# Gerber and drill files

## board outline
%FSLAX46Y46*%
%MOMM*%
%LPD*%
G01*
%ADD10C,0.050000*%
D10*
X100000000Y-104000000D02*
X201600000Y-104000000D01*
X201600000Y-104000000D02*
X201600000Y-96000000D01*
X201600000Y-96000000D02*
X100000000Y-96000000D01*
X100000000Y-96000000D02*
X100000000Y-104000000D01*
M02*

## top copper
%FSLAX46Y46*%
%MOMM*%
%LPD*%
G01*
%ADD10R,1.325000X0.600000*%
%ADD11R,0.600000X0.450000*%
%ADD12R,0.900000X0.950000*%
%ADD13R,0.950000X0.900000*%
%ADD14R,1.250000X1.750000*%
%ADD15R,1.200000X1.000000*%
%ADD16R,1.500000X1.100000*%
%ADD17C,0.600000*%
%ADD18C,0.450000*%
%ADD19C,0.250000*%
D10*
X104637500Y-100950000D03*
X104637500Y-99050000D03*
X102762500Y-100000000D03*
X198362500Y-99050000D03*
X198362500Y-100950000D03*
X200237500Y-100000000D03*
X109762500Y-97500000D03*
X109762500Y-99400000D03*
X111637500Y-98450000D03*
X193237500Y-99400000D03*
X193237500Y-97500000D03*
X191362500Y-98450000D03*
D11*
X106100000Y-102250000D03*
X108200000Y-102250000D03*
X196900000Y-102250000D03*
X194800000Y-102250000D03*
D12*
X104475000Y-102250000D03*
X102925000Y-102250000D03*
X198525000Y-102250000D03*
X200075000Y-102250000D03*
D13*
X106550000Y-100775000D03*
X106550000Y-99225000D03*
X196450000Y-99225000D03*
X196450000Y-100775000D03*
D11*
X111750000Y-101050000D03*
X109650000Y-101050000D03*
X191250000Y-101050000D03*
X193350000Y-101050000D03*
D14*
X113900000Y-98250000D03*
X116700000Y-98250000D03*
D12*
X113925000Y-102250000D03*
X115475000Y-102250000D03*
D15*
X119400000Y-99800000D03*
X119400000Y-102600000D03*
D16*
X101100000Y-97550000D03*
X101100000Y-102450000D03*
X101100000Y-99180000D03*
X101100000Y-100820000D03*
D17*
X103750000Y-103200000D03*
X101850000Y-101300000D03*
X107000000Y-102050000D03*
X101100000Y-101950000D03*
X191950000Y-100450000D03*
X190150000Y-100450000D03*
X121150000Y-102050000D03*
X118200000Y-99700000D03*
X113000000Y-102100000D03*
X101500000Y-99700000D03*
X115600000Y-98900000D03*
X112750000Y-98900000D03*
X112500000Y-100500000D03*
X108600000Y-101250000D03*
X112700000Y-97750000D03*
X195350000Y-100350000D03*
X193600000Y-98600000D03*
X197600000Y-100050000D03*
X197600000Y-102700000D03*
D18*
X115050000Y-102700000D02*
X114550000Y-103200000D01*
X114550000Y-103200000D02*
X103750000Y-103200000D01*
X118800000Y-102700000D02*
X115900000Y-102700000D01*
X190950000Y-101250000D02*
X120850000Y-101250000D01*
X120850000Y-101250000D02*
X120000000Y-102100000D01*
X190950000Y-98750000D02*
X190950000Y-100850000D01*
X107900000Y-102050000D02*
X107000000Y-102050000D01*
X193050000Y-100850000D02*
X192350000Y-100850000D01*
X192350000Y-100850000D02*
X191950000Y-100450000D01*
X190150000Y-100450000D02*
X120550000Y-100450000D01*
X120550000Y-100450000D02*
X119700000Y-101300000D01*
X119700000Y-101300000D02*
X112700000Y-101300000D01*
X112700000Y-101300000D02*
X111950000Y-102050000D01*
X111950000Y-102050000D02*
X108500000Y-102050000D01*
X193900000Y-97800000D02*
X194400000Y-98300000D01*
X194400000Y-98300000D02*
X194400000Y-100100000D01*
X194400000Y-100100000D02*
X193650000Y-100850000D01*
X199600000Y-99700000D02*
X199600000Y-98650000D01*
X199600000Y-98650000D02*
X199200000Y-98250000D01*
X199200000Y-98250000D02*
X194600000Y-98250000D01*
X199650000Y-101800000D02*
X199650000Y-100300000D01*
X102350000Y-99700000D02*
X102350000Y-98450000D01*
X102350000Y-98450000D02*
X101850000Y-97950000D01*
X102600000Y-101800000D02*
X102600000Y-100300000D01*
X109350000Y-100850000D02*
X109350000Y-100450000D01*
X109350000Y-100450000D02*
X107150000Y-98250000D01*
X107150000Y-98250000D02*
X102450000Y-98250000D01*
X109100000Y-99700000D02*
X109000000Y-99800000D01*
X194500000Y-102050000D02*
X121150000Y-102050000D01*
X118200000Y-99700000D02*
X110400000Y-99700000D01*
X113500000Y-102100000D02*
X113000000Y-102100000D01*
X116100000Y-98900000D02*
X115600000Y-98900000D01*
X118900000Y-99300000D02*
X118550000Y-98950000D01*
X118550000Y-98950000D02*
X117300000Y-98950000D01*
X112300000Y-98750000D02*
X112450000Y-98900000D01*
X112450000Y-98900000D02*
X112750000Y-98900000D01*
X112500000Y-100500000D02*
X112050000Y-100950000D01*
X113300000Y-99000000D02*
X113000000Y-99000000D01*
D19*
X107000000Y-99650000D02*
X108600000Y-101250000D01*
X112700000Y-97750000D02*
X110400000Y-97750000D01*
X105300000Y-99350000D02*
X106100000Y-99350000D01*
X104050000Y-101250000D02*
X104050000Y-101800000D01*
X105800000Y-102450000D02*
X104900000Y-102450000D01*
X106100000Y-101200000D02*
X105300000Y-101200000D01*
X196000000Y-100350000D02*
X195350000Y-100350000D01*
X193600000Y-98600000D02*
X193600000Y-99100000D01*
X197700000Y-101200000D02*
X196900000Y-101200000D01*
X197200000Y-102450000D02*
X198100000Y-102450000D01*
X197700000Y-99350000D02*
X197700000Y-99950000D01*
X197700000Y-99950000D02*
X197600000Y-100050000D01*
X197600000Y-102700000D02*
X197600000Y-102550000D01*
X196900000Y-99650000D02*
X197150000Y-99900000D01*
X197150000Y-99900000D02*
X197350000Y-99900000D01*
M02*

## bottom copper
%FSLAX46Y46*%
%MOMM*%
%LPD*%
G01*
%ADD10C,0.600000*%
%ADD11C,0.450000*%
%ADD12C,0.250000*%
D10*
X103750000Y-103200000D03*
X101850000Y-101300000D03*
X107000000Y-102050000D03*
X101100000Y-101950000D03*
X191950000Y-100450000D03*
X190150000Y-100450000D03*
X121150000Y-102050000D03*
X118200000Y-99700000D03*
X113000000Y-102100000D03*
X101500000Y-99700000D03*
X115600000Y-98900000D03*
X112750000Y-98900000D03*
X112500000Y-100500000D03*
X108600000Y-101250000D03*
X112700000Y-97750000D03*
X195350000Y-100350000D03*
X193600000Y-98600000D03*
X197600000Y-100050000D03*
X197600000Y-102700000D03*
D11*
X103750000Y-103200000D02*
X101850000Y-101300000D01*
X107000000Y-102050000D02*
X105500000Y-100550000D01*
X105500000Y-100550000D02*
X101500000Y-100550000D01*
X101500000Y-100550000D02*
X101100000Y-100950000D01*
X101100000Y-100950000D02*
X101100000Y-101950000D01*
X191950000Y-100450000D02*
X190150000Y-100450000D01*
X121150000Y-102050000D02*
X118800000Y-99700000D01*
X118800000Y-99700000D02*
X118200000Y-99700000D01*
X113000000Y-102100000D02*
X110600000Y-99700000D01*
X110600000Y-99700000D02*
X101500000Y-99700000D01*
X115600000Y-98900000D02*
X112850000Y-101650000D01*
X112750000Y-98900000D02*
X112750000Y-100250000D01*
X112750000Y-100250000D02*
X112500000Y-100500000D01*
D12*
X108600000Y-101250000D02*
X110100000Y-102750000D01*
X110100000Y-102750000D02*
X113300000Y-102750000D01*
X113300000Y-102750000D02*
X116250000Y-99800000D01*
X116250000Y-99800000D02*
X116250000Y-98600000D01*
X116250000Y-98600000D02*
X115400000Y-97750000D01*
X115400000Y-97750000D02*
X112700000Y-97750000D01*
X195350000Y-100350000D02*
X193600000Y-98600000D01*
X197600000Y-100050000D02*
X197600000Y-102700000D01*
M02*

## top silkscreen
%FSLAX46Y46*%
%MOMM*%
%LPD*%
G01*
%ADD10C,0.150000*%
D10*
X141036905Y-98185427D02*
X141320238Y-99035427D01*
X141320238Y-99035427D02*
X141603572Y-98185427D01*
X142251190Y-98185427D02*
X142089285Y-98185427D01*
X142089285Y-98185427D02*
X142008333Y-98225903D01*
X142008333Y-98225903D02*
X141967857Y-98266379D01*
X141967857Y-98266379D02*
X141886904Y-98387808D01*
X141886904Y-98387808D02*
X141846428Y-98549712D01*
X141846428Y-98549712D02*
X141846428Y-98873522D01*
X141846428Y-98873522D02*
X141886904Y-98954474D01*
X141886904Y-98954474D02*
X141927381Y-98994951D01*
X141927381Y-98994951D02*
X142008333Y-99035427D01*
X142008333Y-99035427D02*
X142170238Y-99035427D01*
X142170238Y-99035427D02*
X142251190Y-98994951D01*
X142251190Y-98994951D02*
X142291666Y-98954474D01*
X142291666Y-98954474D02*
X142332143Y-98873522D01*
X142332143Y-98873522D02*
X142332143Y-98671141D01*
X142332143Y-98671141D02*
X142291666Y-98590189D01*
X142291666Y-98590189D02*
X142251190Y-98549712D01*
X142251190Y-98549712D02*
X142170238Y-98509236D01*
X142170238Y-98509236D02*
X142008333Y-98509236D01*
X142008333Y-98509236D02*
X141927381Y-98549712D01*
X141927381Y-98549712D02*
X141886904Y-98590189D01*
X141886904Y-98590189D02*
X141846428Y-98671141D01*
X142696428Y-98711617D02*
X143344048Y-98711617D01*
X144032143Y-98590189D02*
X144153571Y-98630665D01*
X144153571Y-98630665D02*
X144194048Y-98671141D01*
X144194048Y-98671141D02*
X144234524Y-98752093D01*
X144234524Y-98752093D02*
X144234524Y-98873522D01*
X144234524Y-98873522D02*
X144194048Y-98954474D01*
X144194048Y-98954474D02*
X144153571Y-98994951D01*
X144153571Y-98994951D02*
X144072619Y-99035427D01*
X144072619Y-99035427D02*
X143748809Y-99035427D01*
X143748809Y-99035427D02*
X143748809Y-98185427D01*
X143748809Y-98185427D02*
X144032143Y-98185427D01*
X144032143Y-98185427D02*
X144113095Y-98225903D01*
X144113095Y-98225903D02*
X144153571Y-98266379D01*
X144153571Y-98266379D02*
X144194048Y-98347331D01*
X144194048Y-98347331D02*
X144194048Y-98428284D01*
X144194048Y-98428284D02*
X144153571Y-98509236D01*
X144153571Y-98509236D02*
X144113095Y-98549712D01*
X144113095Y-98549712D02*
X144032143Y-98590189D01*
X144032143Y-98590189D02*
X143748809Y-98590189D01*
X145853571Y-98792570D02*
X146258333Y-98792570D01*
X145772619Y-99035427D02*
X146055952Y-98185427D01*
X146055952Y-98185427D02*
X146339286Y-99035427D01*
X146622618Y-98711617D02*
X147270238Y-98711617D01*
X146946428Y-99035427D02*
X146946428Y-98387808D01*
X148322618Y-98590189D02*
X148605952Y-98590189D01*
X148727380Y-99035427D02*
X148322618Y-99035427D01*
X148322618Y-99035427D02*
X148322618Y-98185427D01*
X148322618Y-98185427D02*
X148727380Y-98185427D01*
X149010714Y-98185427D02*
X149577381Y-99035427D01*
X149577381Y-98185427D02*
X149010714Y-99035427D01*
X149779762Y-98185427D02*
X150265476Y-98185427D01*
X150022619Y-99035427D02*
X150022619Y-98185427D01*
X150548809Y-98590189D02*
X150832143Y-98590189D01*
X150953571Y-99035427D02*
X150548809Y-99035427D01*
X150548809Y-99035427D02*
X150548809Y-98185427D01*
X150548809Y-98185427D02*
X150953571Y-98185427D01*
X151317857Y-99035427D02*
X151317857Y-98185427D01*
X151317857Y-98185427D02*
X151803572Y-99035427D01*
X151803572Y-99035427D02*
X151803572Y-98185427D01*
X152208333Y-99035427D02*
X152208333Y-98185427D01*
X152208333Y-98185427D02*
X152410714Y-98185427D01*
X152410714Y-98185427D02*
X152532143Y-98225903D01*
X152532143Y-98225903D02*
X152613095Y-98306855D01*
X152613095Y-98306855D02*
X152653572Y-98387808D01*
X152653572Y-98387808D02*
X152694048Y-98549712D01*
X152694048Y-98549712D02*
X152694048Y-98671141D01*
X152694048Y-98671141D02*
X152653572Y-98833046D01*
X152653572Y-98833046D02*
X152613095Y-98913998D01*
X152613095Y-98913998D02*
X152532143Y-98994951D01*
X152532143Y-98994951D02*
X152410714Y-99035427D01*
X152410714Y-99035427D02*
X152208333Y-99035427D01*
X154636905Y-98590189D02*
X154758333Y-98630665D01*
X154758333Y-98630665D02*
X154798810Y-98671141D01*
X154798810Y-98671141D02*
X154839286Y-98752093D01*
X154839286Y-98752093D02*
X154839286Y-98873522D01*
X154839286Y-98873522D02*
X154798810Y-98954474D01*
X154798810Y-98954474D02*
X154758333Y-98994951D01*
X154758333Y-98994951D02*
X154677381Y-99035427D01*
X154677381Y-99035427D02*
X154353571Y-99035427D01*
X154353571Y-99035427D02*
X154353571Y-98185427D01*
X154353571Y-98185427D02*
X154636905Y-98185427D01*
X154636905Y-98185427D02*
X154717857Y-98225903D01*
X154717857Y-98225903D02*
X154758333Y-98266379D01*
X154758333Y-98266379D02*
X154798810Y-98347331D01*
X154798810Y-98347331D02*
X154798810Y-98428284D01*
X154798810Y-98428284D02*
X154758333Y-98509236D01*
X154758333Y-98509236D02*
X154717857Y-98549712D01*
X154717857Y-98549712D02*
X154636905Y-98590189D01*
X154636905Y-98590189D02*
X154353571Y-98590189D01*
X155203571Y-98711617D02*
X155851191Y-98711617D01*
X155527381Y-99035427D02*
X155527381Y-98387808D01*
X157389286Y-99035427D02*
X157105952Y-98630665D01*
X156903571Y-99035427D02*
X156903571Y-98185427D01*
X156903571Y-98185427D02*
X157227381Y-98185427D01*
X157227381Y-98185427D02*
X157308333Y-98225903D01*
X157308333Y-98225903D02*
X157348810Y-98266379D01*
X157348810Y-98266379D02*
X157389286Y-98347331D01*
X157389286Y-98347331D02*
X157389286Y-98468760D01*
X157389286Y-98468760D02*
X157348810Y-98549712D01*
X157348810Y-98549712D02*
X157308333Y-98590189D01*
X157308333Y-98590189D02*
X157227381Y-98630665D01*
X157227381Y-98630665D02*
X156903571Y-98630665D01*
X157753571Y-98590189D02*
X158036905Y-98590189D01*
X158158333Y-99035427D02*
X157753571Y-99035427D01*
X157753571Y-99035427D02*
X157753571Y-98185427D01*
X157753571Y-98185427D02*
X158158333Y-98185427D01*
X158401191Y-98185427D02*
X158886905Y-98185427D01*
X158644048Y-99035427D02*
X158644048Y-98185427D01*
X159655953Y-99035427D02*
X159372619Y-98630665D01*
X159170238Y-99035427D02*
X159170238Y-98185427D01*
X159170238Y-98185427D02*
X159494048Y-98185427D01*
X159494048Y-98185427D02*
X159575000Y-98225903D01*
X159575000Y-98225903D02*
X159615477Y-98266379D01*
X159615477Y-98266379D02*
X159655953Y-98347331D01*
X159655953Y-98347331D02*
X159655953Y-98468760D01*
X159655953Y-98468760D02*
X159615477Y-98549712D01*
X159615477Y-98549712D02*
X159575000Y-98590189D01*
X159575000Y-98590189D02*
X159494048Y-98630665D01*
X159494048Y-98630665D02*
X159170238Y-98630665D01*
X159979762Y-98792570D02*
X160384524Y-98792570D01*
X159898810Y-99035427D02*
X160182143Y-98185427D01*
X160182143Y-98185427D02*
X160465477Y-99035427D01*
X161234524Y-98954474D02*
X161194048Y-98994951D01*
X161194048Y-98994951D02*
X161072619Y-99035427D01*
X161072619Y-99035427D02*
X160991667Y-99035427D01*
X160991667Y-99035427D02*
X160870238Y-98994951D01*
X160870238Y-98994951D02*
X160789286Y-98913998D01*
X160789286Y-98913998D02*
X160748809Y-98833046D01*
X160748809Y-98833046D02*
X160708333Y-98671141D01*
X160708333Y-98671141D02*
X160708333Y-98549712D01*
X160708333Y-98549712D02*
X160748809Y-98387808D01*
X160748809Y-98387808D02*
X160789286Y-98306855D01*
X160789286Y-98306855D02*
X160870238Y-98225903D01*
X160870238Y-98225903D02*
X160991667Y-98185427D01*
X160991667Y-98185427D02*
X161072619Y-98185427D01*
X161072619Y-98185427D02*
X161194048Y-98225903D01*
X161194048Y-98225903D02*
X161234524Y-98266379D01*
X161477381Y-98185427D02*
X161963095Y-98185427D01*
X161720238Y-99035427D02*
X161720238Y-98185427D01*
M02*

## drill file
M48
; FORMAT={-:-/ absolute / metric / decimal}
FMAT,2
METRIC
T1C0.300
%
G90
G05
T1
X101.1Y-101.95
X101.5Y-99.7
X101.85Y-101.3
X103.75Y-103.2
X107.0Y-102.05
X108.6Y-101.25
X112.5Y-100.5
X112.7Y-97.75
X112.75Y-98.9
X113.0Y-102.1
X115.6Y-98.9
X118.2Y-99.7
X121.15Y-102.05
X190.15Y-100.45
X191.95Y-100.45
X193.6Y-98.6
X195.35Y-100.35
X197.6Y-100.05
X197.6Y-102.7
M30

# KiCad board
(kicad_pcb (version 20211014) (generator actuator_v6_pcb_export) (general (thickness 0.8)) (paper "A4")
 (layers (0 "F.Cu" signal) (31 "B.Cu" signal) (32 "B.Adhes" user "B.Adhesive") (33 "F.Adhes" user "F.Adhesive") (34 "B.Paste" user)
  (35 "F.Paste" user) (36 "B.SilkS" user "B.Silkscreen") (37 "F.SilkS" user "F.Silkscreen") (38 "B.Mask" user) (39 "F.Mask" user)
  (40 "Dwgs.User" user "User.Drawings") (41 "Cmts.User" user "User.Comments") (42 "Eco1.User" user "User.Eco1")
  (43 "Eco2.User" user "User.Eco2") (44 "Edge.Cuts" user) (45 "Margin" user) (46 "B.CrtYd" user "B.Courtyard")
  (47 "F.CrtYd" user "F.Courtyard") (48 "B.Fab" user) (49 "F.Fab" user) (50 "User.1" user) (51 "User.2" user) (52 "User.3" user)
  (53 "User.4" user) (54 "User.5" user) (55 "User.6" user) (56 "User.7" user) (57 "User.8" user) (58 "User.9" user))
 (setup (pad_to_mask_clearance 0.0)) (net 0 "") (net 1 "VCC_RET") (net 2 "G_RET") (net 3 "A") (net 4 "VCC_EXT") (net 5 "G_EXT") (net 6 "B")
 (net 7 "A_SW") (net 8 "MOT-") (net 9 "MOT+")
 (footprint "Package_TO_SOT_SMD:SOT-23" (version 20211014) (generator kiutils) (layer "F.Cu") (at 103.7 100.0 180)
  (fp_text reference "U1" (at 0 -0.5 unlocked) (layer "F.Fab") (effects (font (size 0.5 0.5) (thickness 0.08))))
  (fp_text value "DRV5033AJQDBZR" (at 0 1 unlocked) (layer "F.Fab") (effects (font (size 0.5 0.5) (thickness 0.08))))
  (pad "1" smd rect (at -0.9375 -0.95 180) (size 1.325 0.6) (layers "F.Cu" "F.Mask" "F.Paste") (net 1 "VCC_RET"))
  (pad "2" smd rect (at -0.9375 0.95 180) (size 1.325 0.6) (layers "F.Cu" "F.Mask" "F.Paste") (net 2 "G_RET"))
  (pad "3" smd rect (at 0.9375 0.0 180) (size 1.325 0.6) (layers "F.Cu" "F.Mask" "F.Paste") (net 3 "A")))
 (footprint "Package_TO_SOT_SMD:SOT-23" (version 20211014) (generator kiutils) (layer "F.Cu") (at 199.3 100.0)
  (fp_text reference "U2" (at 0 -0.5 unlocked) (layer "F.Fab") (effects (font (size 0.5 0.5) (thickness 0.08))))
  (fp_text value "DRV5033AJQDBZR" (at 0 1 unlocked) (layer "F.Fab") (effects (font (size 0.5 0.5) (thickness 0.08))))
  (pad "1" smd rect (at -0.9375 -0.95) (size 1.325 0.6) (layers "F.Cu" "F.Mask" "F.Paste") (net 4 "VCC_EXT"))
  (pad "2" smd rect (at -0.9375 0.95) (size 1.325 0.6) (layers "F.Cu" "F.Mask" "F.Paste") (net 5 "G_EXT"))
  (pad "3" smd rect (at 0.9375 0.0) (size 1.325 0.6) (layers "F.Cu" "F.Mask" "F.Paste") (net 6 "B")))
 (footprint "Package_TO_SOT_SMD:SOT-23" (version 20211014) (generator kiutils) (layer "F.Cu") (at 110.7 98.45)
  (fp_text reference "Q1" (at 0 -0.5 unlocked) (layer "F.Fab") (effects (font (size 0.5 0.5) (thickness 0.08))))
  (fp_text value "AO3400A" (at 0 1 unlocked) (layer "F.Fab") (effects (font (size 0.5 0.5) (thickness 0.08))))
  (pad "1" smd rect (at -0.9375 -0.95) (size 1.325 0.6) (layers "F.Cu" "F.Mask" "F.Paste") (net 2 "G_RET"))
  (pad "2" smd rect (at -0.9375 0.95) (size 1.325 0.6) (layers "F.Cu" "F.Mask" "F.Paste") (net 3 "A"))
  (pad "3" smd rect (at 0.9375 0.0) (size 1.325 0.6) (layers "F.Cu" "F.Mask" "F.Paste") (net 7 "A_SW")))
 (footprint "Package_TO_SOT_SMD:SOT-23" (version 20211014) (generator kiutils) (layer "F.Cu") (at 192.3 98.45 180)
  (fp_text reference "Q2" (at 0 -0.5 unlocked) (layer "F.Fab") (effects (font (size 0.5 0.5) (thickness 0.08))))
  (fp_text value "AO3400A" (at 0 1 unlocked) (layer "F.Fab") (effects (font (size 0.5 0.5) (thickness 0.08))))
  (pad "1" smd rect (at -0.9375 -0.95 180) (size 1.325 0.6) (layers "F.Cu" "F.Mask" "F.Paste") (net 5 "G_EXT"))
  (pad "2" smd rect (at -0.9375 0.95 180) (size 1.325 0.6) (layers "F.Cu" "F.Mask" "F.Paste") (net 6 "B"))
  (pad "3" smd rect (at 0.9375 0.0 180) (size 1.325 0.6) (layers "F.Cu" "F.Mask" "F.Paste") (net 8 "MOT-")))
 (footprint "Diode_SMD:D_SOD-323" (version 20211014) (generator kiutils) (layer "F.Cu") (at 107.15 102.25)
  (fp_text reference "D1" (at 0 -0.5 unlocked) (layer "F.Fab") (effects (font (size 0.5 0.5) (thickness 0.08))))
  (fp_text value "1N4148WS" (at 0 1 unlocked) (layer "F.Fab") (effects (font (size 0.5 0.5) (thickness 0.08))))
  (pad "1" smd rect (at -1.05 0.0) (size 0.6 0.45) (layers "F.Cu" "F.Mask" "F.Paste") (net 1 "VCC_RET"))
  (pad "2" smd rect (at 1.05 0.0) (size 0.6 0.45) (layers "F.Cu" "F.Mask" "F.Paste") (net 6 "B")))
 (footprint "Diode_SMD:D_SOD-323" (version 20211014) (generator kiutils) (layer "F.Cu") (at 195.85 102.25 180)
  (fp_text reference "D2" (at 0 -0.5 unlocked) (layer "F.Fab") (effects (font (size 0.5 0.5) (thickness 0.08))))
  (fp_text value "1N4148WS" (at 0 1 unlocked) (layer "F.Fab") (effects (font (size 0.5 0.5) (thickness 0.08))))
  (pad "1" smd rect (at -1.05 0.0 180) (size 0.6 0.45) (layers "F.Cu" "F.Mask" "F.Paste") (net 4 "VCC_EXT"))
  (pad "2" smd rect (at 1.05 0.0 180) (size 0.6 0.45) (layers "F.Cu" "F.Mask" "F.Paste") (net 3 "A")))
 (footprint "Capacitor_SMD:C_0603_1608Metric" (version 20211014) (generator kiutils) (layer "F.Cu") (at 103.7 102.25 180)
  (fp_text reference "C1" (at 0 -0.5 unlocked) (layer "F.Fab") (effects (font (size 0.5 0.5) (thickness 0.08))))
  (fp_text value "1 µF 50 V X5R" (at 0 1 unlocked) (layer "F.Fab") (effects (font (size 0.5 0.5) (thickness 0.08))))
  (pad "1" smd rect (at -0.775 0.0 180) (size 0.9 0.95) (layers "F.Cu" "F.Mask" "F.Paste") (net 1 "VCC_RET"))
  (pad "2" smd rect (at 0.775 0.0 180) (size 0.9 0.95) (layers "F.Cu" "F.Mask" "F.Paste") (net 3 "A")))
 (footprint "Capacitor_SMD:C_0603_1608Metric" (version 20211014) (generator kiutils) (layer "F.Cu") (at 199.3 102.25)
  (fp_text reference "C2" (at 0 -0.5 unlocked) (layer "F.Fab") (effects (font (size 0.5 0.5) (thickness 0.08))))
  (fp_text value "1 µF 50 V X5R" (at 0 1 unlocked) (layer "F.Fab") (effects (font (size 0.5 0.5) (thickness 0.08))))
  (pad "1" smd rect (at -0.775 0.0) (size 0.9 0.95) (layers "F.Cu" "F.Mask" "F.Paste") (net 4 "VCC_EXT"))
  (pad "2" smd rect (at 0.775 0.0) (size 0.9 0.95) (layers "F.Cu" "F.Mask" "F.Paste") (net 6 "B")))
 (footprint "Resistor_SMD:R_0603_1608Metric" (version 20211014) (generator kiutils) (layer "F.Cu") (at 106.55 100.0 90)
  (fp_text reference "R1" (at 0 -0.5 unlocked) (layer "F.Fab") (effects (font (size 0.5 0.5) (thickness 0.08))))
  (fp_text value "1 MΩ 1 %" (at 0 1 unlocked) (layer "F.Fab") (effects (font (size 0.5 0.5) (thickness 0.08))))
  (pad "1" smd rect (at -0.775 0.0 90) (size 0.9 0.95) (layers "F.Cu" "F.Mask" "F.Paste") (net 1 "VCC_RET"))
  (pad "2" smd rect (at 0.775 0.0 90) (size 0.9 0.95) (layers "F.Cu" "F.Mask" "F.Paste") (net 2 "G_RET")))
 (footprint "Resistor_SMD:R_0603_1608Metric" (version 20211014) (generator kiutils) (layer "F.Cu") (at 196.45 100.0 270)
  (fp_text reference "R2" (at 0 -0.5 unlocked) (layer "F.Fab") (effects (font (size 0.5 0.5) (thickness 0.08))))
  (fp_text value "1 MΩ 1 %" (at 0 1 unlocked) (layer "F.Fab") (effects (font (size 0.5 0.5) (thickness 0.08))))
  (pad "1" smd rect (at -0.775 0.0 270) (size 0.9 0.95) (layers "F.Cu" "F.Mask" "F.Paste") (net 4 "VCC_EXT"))
  (pad "2" smd rect (at 0.775 0.0 270) (size 0.9 0.95) (layers "F.Cu" "F.Mask" "F.Paste") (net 5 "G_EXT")))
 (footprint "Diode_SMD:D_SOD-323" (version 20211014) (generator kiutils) (layer "F.Cu") (at 110.7 101.05 180)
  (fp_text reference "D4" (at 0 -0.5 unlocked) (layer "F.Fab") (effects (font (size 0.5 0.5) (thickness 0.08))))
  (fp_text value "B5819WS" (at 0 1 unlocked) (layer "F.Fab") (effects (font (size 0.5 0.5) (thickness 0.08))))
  (pad "1" smd rect (at -1.05 0.0 180) (size 0.6 0.45) (layers "F.Cu" "F.Mask" "F.Paste") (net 7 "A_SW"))
  (pad "2" smd rect (at 1.05 0.0 180) (size 0.6 0.45) (layers "F.Cu" "F.Mask" "F.Paste") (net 3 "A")))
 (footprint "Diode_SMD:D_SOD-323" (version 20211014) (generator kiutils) (layer "F.Cu") (at 192.3 101.05)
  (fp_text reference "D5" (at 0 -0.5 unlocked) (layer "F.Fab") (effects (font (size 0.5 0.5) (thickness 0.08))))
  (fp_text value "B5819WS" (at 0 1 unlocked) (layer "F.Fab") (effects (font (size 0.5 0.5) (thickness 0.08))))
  (pad "1" smd rect (at -1.05 0.0) (size 0.6 0.45) (layers "F.Cu" "F.Mask" "F.Paste") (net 8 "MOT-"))
  (pad "2" smd rect (at 1.05 0.0) (size 0.6 0.45) (layers "F.Cu" "F.Mask" "F.Paste") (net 6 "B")))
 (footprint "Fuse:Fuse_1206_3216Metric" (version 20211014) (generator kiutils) (layer "F.Cu") (at 115.3 98.25)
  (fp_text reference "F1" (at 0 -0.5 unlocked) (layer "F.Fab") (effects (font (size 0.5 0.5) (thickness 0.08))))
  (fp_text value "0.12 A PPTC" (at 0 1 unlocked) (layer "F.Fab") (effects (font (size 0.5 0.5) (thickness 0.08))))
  (pad "1" smd rect (at -1.4 0.0) (size 1.25 1.75) (layers "F.Cu" "F.Mask" "F.Paste") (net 7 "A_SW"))
  (pad "2" smd rect (at 1.4 0.0) (size 1.25 1.75) (layers "F.Cu" "F.Mask" "F.Paste") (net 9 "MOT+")))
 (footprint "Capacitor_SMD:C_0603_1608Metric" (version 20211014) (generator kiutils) (layer "F.Cu") (at 114.7 102.25)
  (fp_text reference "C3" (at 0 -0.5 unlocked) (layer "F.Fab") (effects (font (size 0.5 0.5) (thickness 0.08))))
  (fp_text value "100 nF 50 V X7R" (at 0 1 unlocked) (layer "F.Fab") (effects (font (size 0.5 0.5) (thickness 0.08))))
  (pad "1" smd rect (at -0.775 0.0) (size 0.9 0.95) (layers "F.Cu" "F.Mask" "F.Paste") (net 9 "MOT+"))
  (pad "2" smd rect (at 0.775 0.0) (size 0.9 0.95) (layers "F.Cu" "F.Mask" "F.Paste") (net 8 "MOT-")))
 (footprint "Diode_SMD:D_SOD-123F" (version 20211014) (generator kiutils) (layer "F.Cu") (at 119.4 101.2 270)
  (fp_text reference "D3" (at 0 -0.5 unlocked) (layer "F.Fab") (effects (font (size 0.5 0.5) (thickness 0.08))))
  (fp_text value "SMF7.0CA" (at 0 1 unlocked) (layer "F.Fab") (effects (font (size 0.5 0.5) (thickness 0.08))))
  (pad "1" smd rect (at -1.4 0.0 270) (size 1.0 1.2) (layers "F.Cu" "F.Mask" "F.Paste") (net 9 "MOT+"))
  (pad "2" smd rect (at 1.4 0.0 270) (size 1.0 1.2) (layers "F.Cu" "F.Mask" "F.Paste") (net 8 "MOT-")))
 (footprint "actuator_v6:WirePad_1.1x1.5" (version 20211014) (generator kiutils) (layer "F.Cu") (at 101.1 97.55)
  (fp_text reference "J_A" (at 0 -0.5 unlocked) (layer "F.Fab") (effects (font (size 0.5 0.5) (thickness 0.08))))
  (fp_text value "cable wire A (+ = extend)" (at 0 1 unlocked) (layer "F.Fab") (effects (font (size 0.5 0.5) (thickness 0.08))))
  (pad "1" smd rect (at 0.0 0.0) (size 1.5 1.1) (layers "F.Cu" "F.Mask") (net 3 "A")))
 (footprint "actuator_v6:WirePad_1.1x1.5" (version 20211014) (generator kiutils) (layer "F.Cu") (at 101.1 102.45)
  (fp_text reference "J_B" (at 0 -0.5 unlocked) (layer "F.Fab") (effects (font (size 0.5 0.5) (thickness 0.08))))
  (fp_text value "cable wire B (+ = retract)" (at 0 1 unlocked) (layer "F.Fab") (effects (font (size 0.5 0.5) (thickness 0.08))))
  (pad "1" smd rect (at 0.0 0.0) (size 1.5 1.1) (layers "F.Cu" "F.Mask") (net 6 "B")))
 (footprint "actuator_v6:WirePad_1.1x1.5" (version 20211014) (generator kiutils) (layer "F.Cu") (at 101.1 99.18)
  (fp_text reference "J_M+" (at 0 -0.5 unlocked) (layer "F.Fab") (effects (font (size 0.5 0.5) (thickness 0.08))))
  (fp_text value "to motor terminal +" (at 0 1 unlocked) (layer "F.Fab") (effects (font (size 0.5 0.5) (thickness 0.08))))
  (pad "1" smd rect (at 0.0 0.0) (size 1.5 1.1) (layers "F.Cu" "F.Mask") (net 9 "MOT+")))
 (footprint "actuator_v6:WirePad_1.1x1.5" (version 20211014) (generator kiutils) (layer "F.Cu") (at 101.1 100.82)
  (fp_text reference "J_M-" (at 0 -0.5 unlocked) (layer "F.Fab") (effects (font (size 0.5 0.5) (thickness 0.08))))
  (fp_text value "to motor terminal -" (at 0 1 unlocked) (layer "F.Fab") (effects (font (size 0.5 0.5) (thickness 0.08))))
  (pad "1" smd rect (at 0.0 0.0) (size 1.5 1.1) (layers "F.Cu" "F.Mask") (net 8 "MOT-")))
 (gr_line (start 100.0 104.0) (end 201.6 104.0) (layer "Edge.Cuts") (width 0.05))
 (gr_line (start 201.6 104.0) (end 201.6 96.0) (layer "Edge.Cuts") (width 0.05))
 (gr_line (start 201.6 96.0) (end 100.0 96.0) (layer "Edge.Cuts") (width 0.05))
 (gr_line (start 100.0 96.0) (end 100.0 104.0) (layer "Edge.Cuts") (width 0.05))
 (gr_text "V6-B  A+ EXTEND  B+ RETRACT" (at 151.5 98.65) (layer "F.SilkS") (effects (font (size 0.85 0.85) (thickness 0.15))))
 (segment (start 115.05 102.7) (end 114.55 103.2) (width 0.45) (layer "F.Cu") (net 8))
 (segment (start 114.55 103.2) (end 103.75 103.2) (width 0.45) (layer "F.Cu") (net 8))
 (segment (start 103.75 103.2) (end 101.85 101.3) (width 0.45) (layer "B.Cu") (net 8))
 (segment (start 118.8 102.7) (end 115.9 102.7) (width 0.45) (layer "F.Cu") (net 8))
 (segment (start 190.95 101.25) (end 120.85 101.25) (width 0.45) (layer "F.Cu") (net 8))
 (segment (start 120.85 101.25) (end 120.0 102.1) (width 0.45) (layer "F.Cu") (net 8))
 (segment (start 190.95 98.75) (end 190.95 100.85) (width 0.45) (layer "F.Cu") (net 8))
 (segment (start 107.9 102.05) (end 107.0 102.05) (width 0.45) (layer "F.Cu") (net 6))
 (segment (start 107.0 102.05) (end 105.5 100.55) (width 0.45) (layer "B.Cu") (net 6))
 (segment (start 105.5 100.55) (end 101.5 100.55) (width 0.45) (layer "B.Cu") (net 6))
 (segment (start 101.5 100.55) (end 101.1 100.95) (width 0.45) (layer "B.Cu") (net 6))
 (segment (start 101.1 100.95) (end 101.1 101.95) (width 0.45) (layer "B.Cu") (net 6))
 (segment (start 193.05 100.85) (end 192.35 100.85) (width 0.45) (layer "F.Cu") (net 6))
 (segment (start 192.35 100.85) (end 191.95 100.45) (width 0.45) (layer "F.Cu") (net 6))
 (segment (start 191.95 100.45) (end 190.15 100.45) (width 0.45) (layer "B.Cu") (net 6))
 (segment (start 190.15 100.45) (end 120.55 100.45) (width 0.45) (layer "F.Cu") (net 6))
 (segment (start 120.55 100.45) (end 119.7 101.3) (width 0.45) (layer "F.Cu") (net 6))
 (segment (start 119.7 101.3) (end 112.7 101.3) (width 0.45) (layer "F.Cu") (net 6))
 (segment (start 112.7 101.3) (end 111.95 102.05) (width 0.45) (layer "F.Cu") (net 6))
 (segment (start 111.95 102.05) (end 108.5 102.05) (width 0.45) (layer "F.Cu") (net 6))
 (segment (start 193.9 97.8) (end 194.4 98.3) (width 0.45) (layer "F.Cu") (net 6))
 (segment (start 194.4 98.3) (end 194.4 100.1) (width 0.45) (layer "F.Cu") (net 6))
 (segment (start 194.4 100.1) (end 193.65 100.85) (width 0.45) (layer "F.Cu") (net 6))
 (segment (start 199.6 99.7) (end 199.6 98.65) (width 0.45) (layer "F.Cu") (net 6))
 (segment (start 199.6 98.65) (end 199.2 98.25) (width 0.45) (layer "F.Cu") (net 6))
 (segment (start 199.2 98.25) (end 194.6 98.25) (width 0.45) (layer "F.Cu") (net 6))
 (segment (start 199.65 101.8) (end 199.65 100.3) (width 0.45) (layer "F.Cu") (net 6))
 (segment (start 102.35 99.7) (end 102.35 98.45) (width 0.45) (layer "F.Cu") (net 3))
 (segment (start 102.35 98.45) (end 101.85 97.95) (width 0.45) (layer "F.Cu") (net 3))
 (segment (start 102.6 101.8) (end 102.6 100.3) (width 0.45) (layer "F.Cu") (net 3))
 (segment (start 109.35 100.85) (end 109.35 100.45) (width 0.45) (layer "F.Cu") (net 3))
 (segment (start 109.35 100.45) (end 107.15 98.25) (width 0.45) (layer "F.Cu") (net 3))
 (segment (start 107.15 98.25) (end 102.45 98.25) (width 0.45) (layer "F.Cu") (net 3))
 (segment (start 109.1 99.7) (end 109.0 99.8) (width 0.45) (layer "F.Cu") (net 3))
 (segment (start 194.5 102.05) (end 121.15 102.05) (width 0.45) (layer "F.Cu") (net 3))
 (segment (start 121.15 102.05) (end 118.8 99.7) (width 0.45) (layer "B.Cu") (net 3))
 (segment (start 118.8 99.7) (end 118.2 99.7) (width 0.45) (layer "B.Cu") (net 3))
 (segment (start 118.2 99.7) (end 110.4 99.7) (width 0.45) (layer "F.Cu") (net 3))
 (segment (start 113.5 102.1) (end 113.0 102.1) (width 0.45) (layer "F.Cu") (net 9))
 (segment (start 113.0 102.1) (end 110.6 99.7) (width 0.45) (layer "B.Cu") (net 9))
 (segment (start 110.6 99.7) (end 101.5 99.7) (width 0.45) (layer "B.Cu") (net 9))
 (segment (start 116.1 98.9) (end 115.6 98.9) (width 0.45) (layer "F.Cu") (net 9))
 (segment (start 115.6 98.9) (end 112.85 101.65) (width 0.45) (layer "B.Cu") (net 9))
 (segment (start 118.9 99.3) (end 118.55 98.95) (width 0.45) (layer "F.Cu") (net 9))
 (segment (start 118.55 98.95) (end 117.3 98.95) (width 0.45) (layer "F.Cu") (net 9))
 (segment (start 112.3 98.75) (end 112.45 98.9) (width 0.45) (layer "F.Cu") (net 7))
 (segment (start 112.45 98.9) (end 112.75 98.9) (width 0.45) (layer "F.Cu") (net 7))
 (segment (start 112.75 98.9) (end 112.75 100.25) (width 0.45) (layer "B.Cu") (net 7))
 (segment (start 112.75 100.25) (end 112.5 100.5) (width 0.45) (layer "B.Cu") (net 7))
 (segment (start 112.5 100.5) (end 112.05 100.95) (width 0.45) (layer "F.Cu") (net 7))
 (segment (start 113.3 99.0) (end 113.0 99.0) (width 0.45) (layer "F.Cu") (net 7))
 (segment (start 107.0 99.65) (end 108.6 101.25) (width 0.25) (layer "F.Cu") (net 2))
 (segment (start 108.6 101.25) (end 110.1 102.75) (width 0.25) (layer "B.Cu") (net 2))
 (segment (start 110.1 102.75) (end 113.3 102.75) (width 0.25) (layer "B.Cu") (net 2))
 (segment (start 113.3 102.75) (end 116.25 99.8) (width 0.25) (layer "B.Cu") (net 2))
 (segment (start 116.25 99.8) (end 116.25 98.6) (width 0.25) (layer "B.Cu") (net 2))
 (segment (start 116.25 98.6) (end 115.4 97.75) (width 0.25) (layer "B.Cu") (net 2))
 (segment (start 115.4 97.75) (end 112.7 97.75) (width 0.25) (layer "B.Cu") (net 2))
 (segment (start 112.7 97.75) (end 110.4 97.75) (width 0.25) (layer "F.Cu") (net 2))
 (segment (start 105.3 99.35) (end 106.1 99.35) (width 0.25) (layer "F.Cu") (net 2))
 (segment (start 104.05 101.25) (end 104.05 101.8) (width 0.25) (layer "F.Cu") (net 1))
 (segment (start 105.8 102.45) (end 104.9 102.45) (width 0.25) (layer "F.Cu") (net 1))
 (segment (start 106.1 101.2) (end 105.3 101.2) (width 0.25) (layer "F.Cu") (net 1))
 (segment (start 196.0 100.35) (end 195.35 100.35) (width 0.25) (layer "F.Cu") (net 5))
 (segment (start 195.35 100.35) (end 193.6 98.6) (width 0.25) (layer "B.Cu") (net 5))
 (segment (start 193.6 98.6) (end 193.6 99.1) (width 0.25) (layer "F.Cu") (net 5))
 (segment (start 197.7 101.2) (end 196.9 101.2) (width 0.25) (layer "F.Cu") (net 5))
 (segment (start 197.2 102.45) (end 198.1 102.45) (width 0.25) (layer "F.Cu") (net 4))
 (segment (start 197.7 99.35) (end 197.7 99.95) (width 0.25) (layer "F.Cu") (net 4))
 (segment (start 197.7 99.95) (end 197.6 100.05) (width 0.25) (layer "F.Cu") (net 4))
 (segment (start 197.6 100.05) (end 197.6 102.7) (width 0.25) (layer "B.Cu") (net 4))
 (segment (start 197.6 102.7) (end 197.6 102.55) (width 0.25) (layer "F.Cu") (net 4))
 (segment (start 196.9 99.65) (end 197.15 99.9) (width 0.25) (layer "F.Cu") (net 4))
 (segment (start 197.15 99.9) (end 197.35 99.9) (width 0.25) (layer "F.Cu") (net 4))
 (via (at 103.75 103.2) (size 0.6) (drill 0.3) (layers "F.Cu" "B.Cu") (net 8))
 (via (at 101.85 101.3) (size 0.6) (drill 0.3) (layers "F.Cu" "B.Cu") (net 8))
 (via (at 107.0 102.05) (size 0.6) (drill 0.3) (layers "F.Cu" "B.Cu") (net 6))
 (via (at 101.1 101.95) (size 0.6) (drill 0.3) (layers "F.Cu" "B.Cu") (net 6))
 (via (at 191.95 100.45) (size 0.6) (drill 0.3) (layers "F.Cu" "B.Cu") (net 6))
 (via (at 190.15 100.45) (size 0.6) (drill 0.3) (layers "F.Cu" "B.Cu") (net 6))
 (via (at 121.15 102.05) (size 0.6) (drill 0.3) (layers "F.Cu" "B.Cu") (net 3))
 (via (at 118.2 99.7) (size 0.6) (drill 0.3) (layers "F.Cu" "B.Cu") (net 3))
 (via (at 113.0 102.1) (size 0.6) (drill 0.3) (layers "F.Cu" "B.Cu") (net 9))
 (via (at 101.5 99.7) (size 0.6) (drill 0.3) (layers "F.Cu" "B.Cu") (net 9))
 (via (at 115.6 98.9) (size 0.6) (drill 0.3) (layers "F.Cu" "B.Cu") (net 9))
 (via (at 112.75 98.9) (size 0.6) (drill 0.3) (layers "F.Cu" "B.Cu") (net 7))
 (via (at 112.5 100.5) (size 0.6) (drill 0.3) (layers "F.Cu" "B.Cu") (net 7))
 (via (at 108.6 101.25) (size 0.6) (drill 0.3) (layers "F.Cu" "B.Cu") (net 2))
 (via (at 112.7 97.75) (size 0.6) (drill 0.3) (layers "F.Cu" "B.Cu") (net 2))
 (via (at 195.35 100.35) (size 0.6) (drill 0.3) (layers "F.Cu" "B.Cu") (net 5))
 (via (at 193.6 98.6) (size 0.6) (drill 0.3) (layers "F.Cu" "B.Cu") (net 5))
 (via (at 197.6 100.05) (size 0.6) (drill 0.3) (layers "F.Cu" "B.Cu") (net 4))
 (via (at 197.6 102.7) (size 0.6) (drill 0.3) (layers "F.Cu" "B.Cu") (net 4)))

